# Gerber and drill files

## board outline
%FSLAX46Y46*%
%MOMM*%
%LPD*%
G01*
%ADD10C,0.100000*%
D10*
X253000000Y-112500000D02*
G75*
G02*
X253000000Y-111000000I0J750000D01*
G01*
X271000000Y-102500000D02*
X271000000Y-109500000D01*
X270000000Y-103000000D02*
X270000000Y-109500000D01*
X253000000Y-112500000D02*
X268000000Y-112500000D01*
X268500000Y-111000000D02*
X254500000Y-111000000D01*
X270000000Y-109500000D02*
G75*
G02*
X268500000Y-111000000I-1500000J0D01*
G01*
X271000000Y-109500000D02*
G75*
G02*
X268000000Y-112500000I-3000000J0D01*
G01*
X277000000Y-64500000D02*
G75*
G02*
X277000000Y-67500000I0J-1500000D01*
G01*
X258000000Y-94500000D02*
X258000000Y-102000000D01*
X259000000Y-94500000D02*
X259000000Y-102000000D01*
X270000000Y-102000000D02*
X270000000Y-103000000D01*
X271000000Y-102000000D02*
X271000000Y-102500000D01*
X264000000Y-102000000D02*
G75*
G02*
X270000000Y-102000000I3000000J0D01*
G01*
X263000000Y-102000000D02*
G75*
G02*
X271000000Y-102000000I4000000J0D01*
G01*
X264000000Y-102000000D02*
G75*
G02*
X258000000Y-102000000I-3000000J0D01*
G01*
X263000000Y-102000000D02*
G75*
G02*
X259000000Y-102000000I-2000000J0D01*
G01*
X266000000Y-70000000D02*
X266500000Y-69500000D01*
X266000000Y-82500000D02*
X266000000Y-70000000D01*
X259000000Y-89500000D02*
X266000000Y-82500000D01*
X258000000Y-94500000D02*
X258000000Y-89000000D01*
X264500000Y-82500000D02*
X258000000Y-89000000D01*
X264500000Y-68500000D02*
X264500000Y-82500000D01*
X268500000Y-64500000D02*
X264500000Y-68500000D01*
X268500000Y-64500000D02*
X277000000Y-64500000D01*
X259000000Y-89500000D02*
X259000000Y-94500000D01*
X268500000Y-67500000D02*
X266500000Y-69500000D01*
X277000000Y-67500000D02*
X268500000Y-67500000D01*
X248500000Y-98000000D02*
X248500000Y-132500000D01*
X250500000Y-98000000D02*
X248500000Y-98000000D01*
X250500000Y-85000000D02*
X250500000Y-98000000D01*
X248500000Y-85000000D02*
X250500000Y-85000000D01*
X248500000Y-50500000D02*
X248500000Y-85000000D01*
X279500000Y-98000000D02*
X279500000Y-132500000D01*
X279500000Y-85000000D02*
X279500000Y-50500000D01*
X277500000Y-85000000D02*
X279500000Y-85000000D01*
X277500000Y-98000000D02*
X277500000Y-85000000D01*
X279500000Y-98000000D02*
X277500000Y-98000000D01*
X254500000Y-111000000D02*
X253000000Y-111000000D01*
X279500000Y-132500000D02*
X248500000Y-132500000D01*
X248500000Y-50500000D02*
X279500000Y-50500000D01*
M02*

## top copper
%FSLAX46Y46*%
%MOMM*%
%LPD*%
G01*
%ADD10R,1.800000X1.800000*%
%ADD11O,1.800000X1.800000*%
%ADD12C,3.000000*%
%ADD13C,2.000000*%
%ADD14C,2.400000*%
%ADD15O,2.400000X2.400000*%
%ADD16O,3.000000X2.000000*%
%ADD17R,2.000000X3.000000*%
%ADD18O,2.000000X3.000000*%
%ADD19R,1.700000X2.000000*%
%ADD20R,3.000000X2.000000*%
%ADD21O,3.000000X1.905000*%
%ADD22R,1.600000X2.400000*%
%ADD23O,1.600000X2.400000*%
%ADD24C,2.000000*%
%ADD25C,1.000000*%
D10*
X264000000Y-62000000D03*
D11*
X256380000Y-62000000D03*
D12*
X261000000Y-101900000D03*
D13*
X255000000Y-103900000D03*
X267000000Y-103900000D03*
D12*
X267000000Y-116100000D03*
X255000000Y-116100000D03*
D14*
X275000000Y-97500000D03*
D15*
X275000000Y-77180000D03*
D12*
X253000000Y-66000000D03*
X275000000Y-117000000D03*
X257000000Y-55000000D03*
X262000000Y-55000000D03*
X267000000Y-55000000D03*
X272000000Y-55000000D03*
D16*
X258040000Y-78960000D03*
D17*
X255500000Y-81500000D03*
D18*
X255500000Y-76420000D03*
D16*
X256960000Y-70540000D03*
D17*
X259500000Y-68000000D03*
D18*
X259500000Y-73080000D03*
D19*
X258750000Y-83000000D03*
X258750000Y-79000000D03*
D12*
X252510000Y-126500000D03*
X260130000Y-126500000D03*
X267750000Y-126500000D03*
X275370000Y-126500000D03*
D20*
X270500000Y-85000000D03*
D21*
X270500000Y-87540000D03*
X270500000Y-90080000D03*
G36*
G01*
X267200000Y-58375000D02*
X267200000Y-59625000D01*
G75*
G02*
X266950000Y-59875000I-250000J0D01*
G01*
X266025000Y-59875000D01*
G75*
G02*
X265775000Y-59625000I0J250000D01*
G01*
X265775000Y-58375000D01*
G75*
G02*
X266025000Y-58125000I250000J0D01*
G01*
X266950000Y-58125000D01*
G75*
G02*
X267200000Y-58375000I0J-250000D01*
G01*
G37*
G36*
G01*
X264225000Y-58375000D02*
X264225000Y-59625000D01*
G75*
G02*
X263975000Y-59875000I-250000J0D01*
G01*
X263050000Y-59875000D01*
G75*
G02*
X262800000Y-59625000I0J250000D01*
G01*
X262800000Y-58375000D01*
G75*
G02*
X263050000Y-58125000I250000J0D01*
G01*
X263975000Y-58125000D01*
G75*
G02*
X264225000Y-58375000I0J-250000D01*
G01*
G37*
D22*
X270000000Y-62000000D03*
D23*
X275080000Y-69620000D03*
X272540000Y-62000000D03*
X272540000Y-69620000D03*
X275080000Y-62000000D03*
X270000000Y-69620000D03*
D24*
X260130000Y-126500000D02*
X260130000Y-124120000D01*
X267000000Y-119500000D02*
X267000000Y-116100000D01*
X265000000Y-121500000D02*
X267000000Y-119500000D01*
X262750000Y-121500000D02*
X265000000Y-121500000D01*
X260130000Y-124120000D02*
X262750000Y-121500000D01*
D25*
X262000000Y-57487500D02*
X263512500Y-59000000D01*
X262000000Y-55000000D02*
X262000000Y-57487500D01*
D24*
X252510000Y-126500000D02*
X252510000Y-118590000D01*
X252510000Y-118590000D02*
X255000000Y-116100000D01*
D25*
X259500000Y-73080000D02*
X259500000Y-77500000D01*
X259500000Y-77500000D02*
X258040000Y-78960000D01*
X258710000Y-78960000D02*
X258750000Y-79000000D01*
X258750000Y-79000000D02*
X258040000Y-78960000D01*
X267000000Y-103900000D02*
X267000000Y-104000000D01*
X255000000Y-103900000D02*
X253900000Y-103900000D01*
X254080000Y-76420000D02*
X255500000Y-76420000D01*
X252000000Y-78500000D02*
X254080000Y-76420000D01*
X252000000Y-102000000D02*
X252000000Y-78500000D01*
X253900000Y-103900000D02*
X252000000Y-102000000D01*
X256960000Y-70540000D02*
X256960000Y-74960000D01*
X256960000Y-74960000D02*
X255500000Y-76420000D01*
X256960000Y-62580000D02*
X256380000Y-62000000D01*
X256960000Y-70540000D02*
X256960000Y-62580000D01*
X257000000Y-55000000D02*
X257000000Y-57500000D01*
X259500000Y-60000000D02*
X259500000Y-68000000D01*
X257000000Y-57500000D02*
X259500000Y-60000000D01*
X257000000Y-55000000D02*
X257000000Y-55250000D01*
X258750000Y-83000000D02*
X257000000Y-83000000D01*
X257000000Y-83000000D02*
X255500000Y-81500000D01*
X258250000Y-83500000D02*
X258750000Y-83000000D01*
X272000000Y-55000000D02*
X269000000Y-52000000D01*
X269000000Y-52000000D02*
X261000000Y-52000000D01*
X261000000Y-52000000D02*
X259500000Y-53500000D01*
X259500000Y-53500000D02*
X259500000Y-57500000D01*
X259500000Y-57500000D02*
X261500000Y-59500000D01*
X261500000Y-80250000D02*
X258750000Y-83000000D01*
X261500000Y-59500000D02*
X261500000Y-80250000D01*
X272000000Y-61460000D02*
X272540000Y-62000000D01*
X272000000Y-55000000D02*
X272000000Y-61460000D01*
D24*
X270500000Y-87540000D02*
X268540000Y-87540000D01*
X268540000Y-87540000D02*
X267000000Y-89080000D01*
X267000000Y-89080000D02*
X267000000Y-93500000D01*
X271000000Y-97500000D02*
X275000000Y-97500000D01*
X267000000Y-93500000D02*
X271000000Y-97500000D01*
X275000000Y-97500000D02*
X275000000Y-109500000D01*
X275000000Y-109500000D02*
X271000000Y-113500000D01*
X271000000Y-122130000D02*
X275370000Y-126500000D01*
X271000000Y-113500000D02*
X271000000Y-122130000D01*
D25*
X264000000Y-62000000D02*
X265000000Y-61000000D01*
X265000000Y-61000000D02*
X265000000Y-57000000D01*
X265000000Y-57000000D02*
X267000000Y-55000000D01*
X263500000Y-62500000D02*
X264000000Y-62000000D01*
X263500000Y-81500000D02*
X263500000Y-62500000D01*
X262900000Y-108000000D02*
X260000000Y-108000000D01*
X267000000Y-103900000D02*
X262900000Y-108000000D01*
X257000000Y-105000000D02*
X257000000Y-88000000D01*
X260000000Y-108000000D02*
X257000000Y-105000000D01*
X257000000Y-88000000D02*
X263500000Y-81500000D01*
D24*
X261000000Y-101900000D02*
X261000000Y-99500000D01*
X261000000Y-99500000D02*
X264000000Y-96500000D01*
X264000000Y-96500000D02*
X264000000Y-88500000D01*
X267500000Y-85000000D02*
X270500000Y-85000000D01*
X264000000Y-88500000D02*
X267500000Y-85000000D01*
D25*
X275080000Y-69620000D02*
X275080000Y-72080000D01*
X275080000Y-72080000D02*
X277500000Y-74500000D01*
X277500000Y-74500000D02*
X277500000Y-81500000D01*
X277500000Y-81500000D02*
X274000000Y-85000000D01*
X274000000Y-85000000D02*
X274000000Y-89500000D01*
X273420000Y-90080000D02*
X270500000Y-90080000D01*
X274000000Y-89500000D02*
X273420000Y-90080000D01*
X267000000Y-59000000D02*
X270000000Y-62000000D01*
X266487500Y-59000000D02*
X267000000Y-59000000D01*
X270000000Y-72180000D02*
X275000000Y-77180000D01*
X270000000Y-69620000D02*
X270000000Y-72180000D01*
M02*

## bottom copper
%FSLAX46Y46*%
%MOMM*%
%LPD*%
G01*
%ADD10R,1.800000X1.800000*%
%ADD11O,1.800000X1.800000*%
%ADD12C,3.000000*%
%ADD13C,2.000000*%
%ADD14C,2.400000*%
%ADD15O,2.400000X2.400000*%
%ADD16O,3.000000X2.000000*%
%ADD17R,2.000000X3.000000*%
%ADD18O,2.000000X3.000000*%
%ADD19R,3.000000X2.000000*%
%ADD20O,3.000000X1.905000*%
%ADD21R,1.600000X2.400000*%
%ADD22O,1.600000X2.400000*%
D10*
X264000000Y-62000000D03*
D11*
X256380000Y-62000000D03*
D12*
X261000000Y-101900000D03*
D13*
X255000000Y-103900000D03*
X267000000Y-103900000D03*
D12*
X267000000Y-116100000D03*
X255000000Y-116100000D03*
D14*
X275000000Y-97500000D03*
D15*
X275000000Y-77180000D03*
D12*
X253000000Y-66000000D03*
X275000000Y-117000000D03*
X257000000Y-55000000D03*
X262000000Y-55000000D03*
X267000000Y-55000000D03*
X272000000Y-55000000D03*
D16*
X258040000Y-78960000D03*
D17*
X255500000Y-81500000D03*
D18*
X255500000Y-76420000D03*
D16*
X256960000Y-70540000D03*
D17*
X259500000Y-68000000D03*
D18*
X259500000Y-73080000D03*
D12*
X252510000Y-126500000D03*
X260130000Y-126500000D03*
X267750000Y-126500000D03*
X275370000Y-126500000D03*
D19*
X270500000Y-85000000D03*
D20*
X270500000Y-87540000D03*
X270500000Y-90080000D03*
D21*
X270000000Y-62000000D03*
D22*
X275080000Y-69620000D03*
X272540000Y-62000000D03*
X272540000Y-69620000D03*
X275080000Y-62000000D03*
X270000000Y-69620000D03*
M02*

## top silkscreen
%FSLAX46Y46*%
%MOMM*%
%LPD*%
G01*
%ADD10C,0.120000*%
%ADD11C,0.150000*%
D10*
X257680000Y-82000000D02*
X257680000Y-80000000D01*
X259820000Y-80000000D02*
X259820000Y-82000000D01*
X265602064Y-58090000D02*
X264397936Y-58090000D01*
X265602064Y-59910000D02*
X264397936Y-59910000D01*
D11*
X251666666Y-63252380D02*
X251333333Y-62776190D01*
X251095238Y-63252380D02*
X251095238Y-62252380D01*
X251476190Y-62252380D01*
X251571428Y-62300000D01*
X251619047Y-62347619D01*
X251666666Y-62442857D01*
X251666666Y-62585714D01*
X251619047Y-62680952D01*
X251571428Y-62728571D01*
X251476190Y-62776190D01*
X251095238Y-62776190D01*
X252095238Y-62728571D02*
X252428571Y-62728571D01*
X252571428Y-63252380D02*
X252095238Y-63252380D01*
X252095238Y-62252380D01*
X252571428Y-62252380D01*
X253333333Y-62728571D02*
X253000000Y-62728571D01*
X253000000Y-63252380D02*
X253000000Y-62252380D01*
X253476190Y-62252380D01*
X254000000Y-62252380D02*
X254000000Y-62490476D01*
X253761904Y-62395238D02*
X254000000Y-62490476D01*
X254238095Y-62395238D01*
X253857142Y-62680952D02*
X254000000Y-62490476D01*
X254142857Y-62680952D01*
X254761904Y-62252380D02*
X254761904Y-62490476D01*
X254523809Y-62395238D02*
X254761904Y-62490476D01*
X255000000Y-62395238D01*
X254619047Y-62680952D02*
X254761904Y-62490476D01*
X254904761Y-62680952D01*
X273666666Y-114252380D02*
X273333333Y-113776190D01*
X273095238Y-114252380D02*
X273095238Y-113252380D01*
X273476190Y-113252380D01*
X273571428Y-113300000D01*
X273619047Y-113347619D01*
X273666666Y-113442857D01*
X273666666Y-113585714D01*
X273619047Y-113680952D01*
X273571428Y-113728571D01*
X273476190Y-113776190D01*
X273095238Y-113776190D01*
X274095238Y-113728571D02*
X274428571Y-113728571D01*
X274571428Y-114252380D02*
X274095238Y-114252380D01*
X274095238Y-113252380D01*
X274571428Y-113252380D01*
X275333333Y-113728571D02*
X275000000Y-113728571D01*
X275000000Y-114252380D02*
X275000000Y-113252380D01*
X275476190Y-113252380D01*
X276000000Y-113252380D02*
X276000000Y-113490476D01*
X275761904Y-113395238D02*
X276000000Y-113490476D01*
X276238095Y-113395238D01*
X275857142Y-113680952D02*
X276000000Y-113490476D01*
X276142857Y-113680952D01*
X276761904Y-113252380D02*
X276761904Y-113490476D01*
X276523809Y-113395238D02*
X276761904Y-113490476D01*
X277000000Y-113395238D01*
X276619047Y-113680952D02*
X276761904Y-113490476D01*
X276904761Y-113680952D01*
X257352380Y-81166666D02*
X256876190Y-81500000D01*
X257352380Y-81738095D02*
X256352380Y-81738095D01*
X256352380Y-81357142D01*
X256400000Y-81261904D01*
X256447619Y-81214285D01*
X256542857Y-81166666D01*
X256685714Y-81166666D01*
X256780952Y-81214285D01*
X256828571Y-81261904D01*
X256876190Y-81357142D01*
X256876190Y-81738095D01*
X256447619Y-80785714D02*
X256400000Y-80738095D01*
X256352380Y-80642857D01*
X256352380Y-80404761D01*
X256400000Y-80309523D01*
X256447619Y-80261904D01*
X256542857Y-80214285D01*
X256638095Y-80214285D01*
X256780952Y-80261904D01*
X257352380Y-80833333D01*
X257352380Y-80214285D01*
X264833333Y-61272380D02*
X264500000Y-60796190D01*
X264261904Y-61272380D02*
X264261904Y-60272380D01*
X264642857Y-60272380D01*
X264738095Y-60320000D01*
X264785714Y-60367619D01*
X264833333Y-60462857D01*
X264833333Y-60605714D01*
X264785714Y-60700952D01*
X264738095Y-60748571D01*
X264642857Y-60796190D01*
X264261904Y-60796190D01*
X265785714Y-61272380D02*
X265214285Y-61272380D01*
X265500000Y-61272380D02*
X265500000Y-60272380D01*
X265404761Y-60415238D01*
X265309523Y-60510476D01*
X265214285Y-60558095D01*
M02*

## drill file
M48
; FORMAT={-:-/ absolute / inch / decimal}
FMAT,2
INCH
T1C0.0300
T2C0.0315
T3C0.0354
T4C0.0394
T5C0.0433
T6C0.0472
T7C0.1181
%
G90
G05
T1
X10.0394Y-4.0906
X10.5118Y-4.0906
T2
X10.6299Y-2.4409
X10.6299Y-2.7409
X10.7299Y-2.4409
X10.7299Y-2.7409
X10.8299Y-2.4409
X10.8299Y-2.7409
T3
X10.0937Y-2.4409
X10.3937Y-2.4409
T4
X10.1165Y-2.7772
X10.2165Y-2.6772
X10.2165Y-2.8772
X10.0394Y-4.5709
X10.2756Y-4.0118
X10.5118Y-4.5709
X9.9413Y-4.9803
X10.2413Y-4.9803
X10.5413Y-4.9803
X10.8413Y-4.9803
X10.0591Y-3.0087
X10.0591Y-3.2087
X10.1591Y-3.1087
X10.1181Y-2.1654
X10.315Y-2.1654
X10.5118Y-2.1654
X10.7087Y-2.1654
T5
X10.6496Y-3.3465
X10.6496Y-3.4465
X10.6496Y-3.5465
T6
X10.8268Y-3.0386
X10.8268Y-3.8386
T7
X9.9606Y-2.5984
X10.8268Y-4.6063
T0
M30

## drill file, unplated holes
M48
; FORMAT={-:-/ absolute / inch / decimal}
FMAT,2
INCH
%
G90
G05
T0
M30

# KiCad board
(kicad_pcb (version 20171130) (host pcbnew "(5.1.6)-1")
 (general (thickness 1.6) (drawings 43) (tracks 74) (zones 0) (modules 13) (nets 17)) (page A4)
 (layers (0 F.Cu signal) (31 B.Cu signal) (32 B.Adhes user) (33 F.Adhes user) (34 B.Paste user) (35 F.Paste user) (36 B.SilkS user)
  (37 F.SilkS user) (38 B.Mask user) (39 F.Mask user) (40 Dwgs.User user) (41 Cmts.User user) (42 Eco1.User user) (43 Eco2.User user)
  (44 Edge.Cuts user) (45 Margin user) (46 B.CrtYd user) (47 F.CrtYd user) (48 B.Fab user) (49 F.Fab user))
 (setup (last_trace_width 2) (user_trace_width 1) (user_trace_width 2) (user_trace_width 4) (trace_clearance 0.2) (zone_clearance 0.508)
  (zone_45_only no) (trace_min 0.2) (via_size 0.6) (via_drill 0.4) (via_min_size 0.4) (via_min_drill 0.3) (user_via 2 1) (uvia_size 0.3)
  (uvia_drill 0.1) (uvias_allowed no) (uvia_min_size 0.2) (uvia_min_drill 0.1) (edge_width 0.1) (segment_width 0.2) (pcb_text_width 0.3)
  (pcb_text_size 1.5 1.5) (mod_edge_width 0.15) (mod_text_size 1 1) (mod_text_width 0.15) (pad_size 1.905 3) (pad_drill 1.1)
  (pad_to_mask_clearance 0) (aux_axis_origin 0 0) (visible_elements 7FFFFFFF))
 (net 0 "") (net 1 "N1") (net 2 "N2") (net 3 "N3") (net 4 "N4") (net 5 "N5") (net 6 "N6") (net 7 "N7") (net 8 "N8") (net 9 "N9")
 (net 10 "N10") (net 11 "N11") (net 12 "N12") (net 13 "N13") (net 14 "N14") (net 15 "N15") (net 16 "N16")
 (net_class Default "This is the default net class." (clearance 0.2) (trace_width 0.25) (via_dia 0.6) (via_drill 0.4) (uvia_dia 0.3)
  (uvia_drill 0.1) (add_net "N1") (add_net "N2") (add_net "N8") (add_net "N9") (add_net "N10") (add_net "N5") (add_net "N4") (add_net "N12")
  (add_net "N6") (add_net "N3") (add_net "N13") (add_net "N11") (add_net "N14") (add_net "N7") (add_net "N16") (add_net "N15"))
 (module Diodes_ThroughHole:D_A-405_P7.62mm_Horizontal (layer B.Cu) (at 264 62 180)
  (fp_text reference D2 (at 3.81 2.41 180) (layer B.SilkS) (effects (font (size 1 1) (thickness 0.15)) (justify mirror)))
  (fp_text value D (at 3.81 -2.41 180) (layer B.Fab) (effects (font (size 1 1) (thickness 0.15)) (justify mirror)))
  (pad 1 thru_hole rect (at 0 0 180) (size 1.8 1.8) (drill 0.9) (layers *.Cu *.Mask) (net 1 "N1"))
  (pad 2 thru_hole oval (at 7.62 0 180) (size 1.8 1.8) (drill 0.9) (layers *.Cu *.Mask) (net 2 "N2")))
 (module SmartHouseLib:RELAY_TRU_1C (layer B.Cu) (at 261 110 270)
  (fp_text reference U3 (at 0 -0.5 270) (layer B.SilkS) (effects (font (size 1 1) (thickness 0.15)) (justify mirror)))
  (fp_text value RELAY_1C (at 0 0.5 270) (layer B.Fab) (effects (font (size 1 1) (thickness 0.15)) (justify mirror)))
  (pad 3 thru_hole circle (at -8.1 0 270) (size 3 3) (drill 1) (layers *.Cu *.Mask) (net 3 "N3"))
  (pad 1 thru_hole circle (at -6.1 6 270) (size 2 2) (drill 0.762) (layers *.Cu *.Mask) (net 2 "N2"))
  (pad 2 thru_hole circle (at -6.1 -6 270) (size 2 2) (drill 0.762) (layers *.Cu *.Mask) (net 1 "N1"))
  (pad 5 thru_hole circle (at 6.1 -6 270) (size 3 3) (drill 1) (layers *.Cu *.Mask) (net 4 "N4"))
  (pad 4 thru_hole circle (at 6.1 6 270) (size 3 3) (drill 1) (layers *.Cu *.Mask) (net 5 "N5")))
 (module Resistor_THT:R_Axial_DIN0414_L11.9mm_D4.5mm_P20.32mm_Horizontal (layer B.Cu) (at 275 97.5 90)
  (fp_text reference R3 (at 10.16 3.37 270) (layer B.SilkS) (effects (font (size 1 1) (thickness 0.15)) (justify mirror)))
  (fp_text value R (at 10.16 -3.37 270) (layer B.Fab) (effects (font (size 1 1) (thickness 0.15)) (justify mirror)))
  (pad 1 thru_hole circle (at 0 0 90) (size 2.4 2.4) (drill 1.2) (layers *.Cu *.Mask) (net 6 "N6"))
  (pad 2 thru_hole oval (at 20.32 0 90) (size 2.4 2.4) (drill 1.2) (layers *.Cu *.Mask) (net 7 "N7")))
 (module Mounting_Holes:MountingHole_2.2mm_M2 (layer F.Cu) (at 253 66)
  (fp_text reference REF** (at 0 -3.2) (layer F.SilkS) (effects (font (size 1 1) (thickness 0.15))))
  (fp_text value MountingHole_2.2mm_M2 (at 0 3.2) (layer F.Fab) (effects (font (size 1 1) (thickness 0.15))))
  (pad 1 thru_hole circle (at 0 0) (size 3 3) (drill 3) (layers *.Cu *.Mask)))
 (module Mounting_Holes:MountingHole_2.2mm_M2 (layer F.Cu) (at 275 117)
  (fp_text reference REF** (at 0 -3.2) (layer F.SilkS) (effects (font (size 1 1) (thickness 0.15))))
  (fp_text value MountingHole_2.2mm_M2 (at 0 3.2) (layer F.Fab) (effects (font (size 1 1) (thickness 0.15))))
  (pad 1 thru_hole circle (at 0 0) (size 3 3) (drill 3) (layers *.Cu *.Mask)))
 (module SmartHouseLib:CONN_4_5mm (layer B.Cu) (at 267 55)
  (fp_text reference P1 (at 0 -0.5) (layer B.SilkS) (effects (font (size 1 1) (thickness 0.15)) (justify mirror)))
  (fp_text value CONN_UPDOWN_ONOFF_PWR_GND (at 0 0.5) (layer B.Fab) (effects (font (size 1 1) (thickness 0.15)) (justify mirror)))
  (pad 1 thru_hole circle (at -10 0) (size 3 3) (drill 1) (layers *.Cu *.Mask) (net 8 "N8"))
  (pad 2 thru_hole circle (at -5 0) (size 3 3) (drill 1) (layers *.Cu *.Mask) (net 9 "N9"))
  (pad 3 thru_hole circle (at 0 0) (size 3 3) (drill 1) (layers *.Cu *.Mask) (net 1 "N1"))
  (pad 4 thru_hole circle (at 5 0) (size 3 3) (drill 1) (layers *.Cu *.Mask) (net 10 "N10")))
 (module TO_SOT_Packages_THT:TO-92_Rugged (layer B.Cu) (at 255.5 81.5 90)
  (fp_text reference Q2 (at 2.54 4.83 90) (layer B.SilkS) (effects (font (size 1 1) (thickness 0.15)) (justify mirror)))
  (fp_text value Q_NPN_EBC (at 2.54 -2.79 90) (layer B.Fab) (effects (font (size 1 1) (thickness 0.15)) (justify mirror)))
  (pad 2 thru_hole oval (at 2.54 2.54) (size 3 2) (drill 1) (layers *.Cu *.Mask) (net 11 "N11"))
  (pad 1 thru_hole rect (at 0 0) (size 2 3) (drill 1) (layers *.Cu *.Mask) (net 10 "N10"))
  (pad 3 thru_hole oval (at 5.08 0) (size 2 3) (drill 1) (layers *.Cu *.Mask) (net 2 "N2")))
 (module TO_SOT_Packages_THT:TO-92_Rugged (layer B.Cu) (at 259.5 68 270)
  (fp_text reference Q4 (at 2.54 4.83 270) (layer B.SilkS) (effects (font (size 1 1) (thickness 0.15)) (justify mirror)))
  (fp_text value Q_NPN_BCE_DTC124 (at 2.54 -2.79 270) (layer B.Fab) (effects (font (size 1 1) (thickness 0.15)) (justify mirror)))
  (pad 2 thru_hole oval (at 2.54 2.54 180) (size 3 2) (drill 1) (layers *.Cu *.Mask) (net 2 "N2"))
  (pad 1 thru_hole rect (at 0 0 180) (size 2 3) (drill 1) (layers *.Cu *.Mask) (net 8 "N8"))
  (pad 3 thru_hole oval (at 5.08 0 180) (size 2 3) (drill 1) (layers *.Cu *.Mask) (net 11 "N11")))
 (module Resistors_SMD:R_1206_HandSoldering (layer F.Cu) (at 258.75 81 90)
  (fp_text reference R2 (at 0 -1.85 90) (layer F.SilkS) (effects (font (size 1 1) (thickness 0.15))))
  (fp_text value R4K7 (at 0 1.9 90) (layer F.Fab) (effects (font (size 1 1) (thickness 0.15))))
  (fp_line (start -1 -1.07) (end 1 -1.07) (layer F.SilkS) (width 0.12))
  (fp_line (start 1 1.07) (end -1 1.07) (layer F.SilkS) (width 0.12))
  (pad 1 smd rect (at -2 0 90) (size 2 1.7) (layers F.Cu F.Paste F.Mask) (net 10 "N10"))
  (pad 2 smd rect (at 2 0 90) (size 2 1.7) (layers F.Cu F.Paste F.Mask) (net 11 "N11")))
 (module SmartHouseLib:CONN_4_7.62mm (layer B.Cu) (at 267.75 126.5)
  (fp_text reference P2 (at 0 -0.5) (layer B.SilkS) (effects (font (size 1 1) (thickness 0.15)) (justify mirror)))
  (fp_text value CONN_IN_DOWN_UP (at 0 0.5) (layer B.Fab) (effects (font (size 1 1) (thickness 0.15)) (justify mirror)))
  (pad 1 thru_hole circle (at -15.24 0) (size 3 3) (drill 1) (layers *.Cu *.Mask) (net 5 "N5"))
  (pad 2 thru_hole circle (at -7.62 0) (size 3 3) (drill 1) (layers *.Cu *.Mask) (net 4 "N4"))
  (pad 3 thru_hole circle (at 0 0) (size 3 3) (drill 1) (layers *.Cu *.Mask) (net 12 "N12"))
  (pad 4 thru_hole circle (at 7.62 0) (size 3 3) (drill 1) (layers *.Cu *.Mask) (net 6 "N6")))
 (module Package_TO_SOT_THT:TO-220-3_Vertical (layer B.Cu) (at 270.5 85 270)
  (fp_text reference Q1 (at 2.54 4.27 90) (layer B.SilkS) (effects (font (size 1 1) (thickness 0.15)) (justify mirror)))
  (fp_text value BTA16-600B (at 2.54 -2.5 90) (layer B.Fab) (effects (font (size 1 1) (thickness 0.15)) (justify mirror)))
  (pad 1 thru_hole rect (at 0 0 270) (size 2 3) (drill 1.1) (layers *.Cu *.Mask) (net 3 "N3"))
  (pad 2 thru_hole oval (at 2.54 0 270) (size 1.905 3) (drill 1.1) (layers *.Cu *.Mask) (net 6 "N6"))
  (pad 3 thru_hole oval (at 5.08 0 270) (size 1.905 3) (drill 1.1) (layers *.Cu *.Mask) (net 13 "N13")))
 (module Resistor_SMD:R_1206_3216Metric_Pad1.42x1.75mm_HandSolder (layer F.Cu) (at 265 59 180)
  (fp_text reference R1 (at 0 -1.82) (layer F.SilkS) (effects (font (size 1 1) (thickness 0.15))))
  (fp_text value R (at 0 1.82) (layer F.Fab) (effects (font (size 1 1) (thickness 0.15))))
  (fp_line (start -0.602064 0.91) (end 0.602064 0.91) (layer F.SilkS) (width 0.12))
  (fp_line (start -0.602064 -0.91) (end 0.602064 -0.91) (layer F.SilkS) (width 0.12))
  (pad 1 smd roundrect (at -1.4875 0 180) (size 1.425 1.75) (layers F.Cu F.Paste F.Mask) (roundrect_rratio 0.175439) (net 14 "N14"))
  (pad 2 smd roundrect (at 1.4875 0 180) (size 1.425 1.75) (layers F.Cu F.Paste F.Mask) (roundrect_rratio 0.175439) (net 9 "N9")))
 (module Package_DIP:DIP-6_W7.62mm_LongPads (layer B.Cu) (at 270 62 270)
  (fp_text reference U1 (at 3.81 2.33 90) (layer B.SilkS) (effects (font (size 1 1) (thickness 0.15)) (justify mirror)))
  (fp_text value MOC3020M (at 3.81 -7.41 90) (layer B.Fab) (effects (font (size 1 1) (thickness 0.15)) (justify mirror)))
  (pad 1 thru_hole rect (at 0 0 270) (size 2.4 1.6) (drill 0.8) (layers *.Cu *.Mask) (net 14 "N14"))
  (pad 4 thru_hole oval (at 7.62 -5.08 270) (size 2.4 1.6) (drill 0.8) (layers *.Cu *.Mask) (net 13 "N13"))
  (pad 2 thru_hole oval (at 0 -2.54 270) (size 2.4 1.6) (drill 0.8) (layers *.Cu *.Mask) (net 10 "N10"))
  (pad 5 thru_hole oval (at 7.62 -2.54 270) (size 2.4 1.6) (drill 0.8) (layers *.Cu *.Mask) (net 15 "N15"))
  (pad 3 thru_hole oval (at 0 -5.08 270) (size 2.4 1.6) (drill 0.8) (layers *.Cu *.Mask) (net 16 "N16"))
  (pad 6 thru_hole oval (at 7.62 0 270) (size 2.4 1.6) (drill 0.8) (layers *.Cu *.Mask) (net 7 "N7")))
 (gr_arc (start 253 111.75) (end 253 111) (angle -180) (layer Edge.Cuts) (width 0.1))
 (gr_line (start 271 102.5) (end 271 109.5) (layer Edge.Cuts) (width 0.1))
 (gr_line (start 270 103) (end 270 109.5) (layer Edge.Cuts) (width 0.1))
 (gr_line (start 253 112.5) (end 268 112.5) (layer Edge.Cuts) (width 0.1))
 (gr_line (start 268.5 111) (end 254.5 111) (layer Edge.Cuts) (width 0.1))
 (gr_arc (start 268.5 109.5) (end 268.5 111) (angle -90) (layer Edge.Cuts) (width 0.1))
 (gr_arc (start 268 109.5) (end 268 112.5) (angle -90) (layer Edge.Cuts) (width 0.1))
 (gr_arc (start 277 66) (end 277 67.5) (angle -180) (layer Edge.Cuts) (width 0.1))
 (gr_line (start 258 94.5) (end 258 102) (layer Edge.Cuts) (width 0.1))
 (gr_line (start 259 94.5) (end 259 102) (layer Edge.Cuts) (width 0.1))
 (gr_line (start 270 102) (end 270 103) (layer Edge.Cuts) (width 0.1))
 (gr_line (start 271 102) (end 271 102.5) (layer Edge.Cuts) (width 0.1))
 (gr_arc (start 267 102) (end 270 102) (angle -180) (layer Edge.Cuts) (width 0.1))
 (gr_arc (start 267 102) (end 271 102) (angle -180) (layer Edge.Cuts) (width 0.1))
 (gr_arc (start 261 102) (end 258 102) (angle -180) (layer Edge.Cuts) (width 0.1))
 (gr_arc (start 261 102) (end 259 102) (angle -180) (layer Edge.Cuts) (width 0.1))
 (gr_line (start 266 70) (end 266.5 69.5) (layer Edge.Cuts) (width 0.1))
 (gr_line (start 266 82.5) (end 266 70) (layer Edge.Cuts) (width 0.1))
 (gr_line (start 259 89.5) (end 266 82.5) (layer Edge.Cuts) (width 0.1))
 (gr_line (start 258 94.5) (end 258 89) (layer Edge.Cuts) (width 0.1))
 (gr_line (start 264.5 82.5) (end 258 89) (layer Edge.Cuts) (width 0.1))
 (gr_line (start 264.5 68.5) (end 264.5 82.5) (layer Edge.Cuts) (width 0.1))
 (gr_line (start 268.5 64.5) (end 264.5 68.5) (layer Edge.Cuts) (width 0.1))
 (gr_line (start 268.5 64.5) (end 277 64.5) (layer Edge.Cuts) (width 0.1))
 (gr_line (start 259 89.5) (end 259 94.5) (layer Edge.Cuts) (width 0.1))
 (gr_line (start 268.5 67.5) (end 266.5 69.5) (layer Edge.Cuts) (width 0.1))
 (gr_line (start 277 67.5) (end 268.5 67.5) (layer Edge.Cuts) (width 0.1))
 (gr_line (start 248.5 98) (end 248.5 132.5) (angle 90) (layer Edge.Cuts) (width 0.1))
 (gr_line (start 250.5 98) (end 248.5 98) (angle 90) (layer Edge.Cuts) (width 0.1))
 (gr_line (start 250.5 85) (end 250.5 98) (angle 90) (layer Edge.Cuts) (width 0.1))
 (gr_line (start 248.5 85) (end 250.5 85) (angle 90) (layer Edge.Cuts) (width 0.1))
 (gr_line (start 248.5 50.5) (end 248.5 85) (angle 90) (layer Edge.Cuts) (width 0.1))
 (gr_line (start 279.5 98) (end 279.5 132.5) (angle 90) (layer Edge.Cuts) (width 0.1))
 (gr_line (start 279.5 85) (end 279.5 50.5) (angle 90) (layer Edge.Cuts) (width 0.1))
 (gr_line (start 277.5 85) (end 279.5 85) (angle 90) (layer Edge.Cuts) (width 0.1))
 (gr_line (start 277.5 98) (end 277.5 85) (angle 90) (layer Edge.Cuts) (width 0.1))
 (gr_line (start 279.5 98) (end 277.5 98) (angle 90) (layer Edge.Cuts) (width 0.1))
 (gr_line (start 254.5 111) (end 253 111) (angle 90) (layer Edge.Cuts) (width 0.1))
 (gr_line (start 279.5 132.5) (end 248.5 132.5) (angle 90) (layer Edge.Cuts) (width 0.1))
 (gr_line (start 248.5 50.5) (end 279.5 50.5) (angle 90) (layer Edge.Cuts) (width 0.1))
 (segment (start 260.13 126.5) (end 260.13 124.12) (width 2) (layer F.Cu) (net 4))
 (segment (start 267 119.5) (end 267 116.1) (width 2) (layer F.Cu) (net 4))
 (segment (start 265 121.5) (end 267 119.5) (width 2) (layer F.Cu) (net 4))
 (segment (start 262.75 121.5) (end 265 121.5) (width 2) (layer F.Cu) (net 4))
 (segment (start 260.13 124.12) (end 262.75 121.5) (width 2) (layer F.Cu) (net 4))
 (segment (start 262 57.4875) (end 263.5125 59) (width 1) (layer F.Cu) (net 9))
 (segment (start 262 55) (end 262 57.4875) (width 1) (layer F.Cu) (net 9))
 (segment (start 252.51 126.5) (end 252.51 118.59) (width 2) (layer F.Cu) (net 5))
 (segment (start 252.51 118.59) (end 255 116.1) (width 2) (layer F.Cu) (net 5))
 (segment (start 259.5 73.08) (end 259.5 77.5) (width 1) (layer F.Cu) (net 11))
 (segment (start 259.5 77.5) (end 258.04 78.96) (width 1) (layer F.Cu) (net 11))
 (segment (start 258.71 78.96) (end 258.75 79) (width 1) (layer F.Cu) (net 11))
 (segment (start 258.75 79) (end 258.04 78.96) (width 1) (layer F.Cu) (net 11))
 (segment (start 267 103.9) (end 267 104) (width 1) (layer F.Cu) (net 1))
 (segment (start 255 103.9) (end 253.9 103.9) (width 1) (layer F.Cu) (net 2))
 (segment (start 254.08 76.42) (end 255.5 76.42) (width 1) (layer F.Cu) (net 2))
 (segment (start 252 78.5) (end 254.08 76.42) (width 1) (layer F.Cu) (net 2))
 (segment (start 252 102) (end 252 78.5) (width 1) (layer F.Cu) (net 2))
 (segment (start 253.9 103.9) (end 252 102) (width 1) (layer F.Cu) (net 2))
 (segment (start 256.96 70.54) (end 256.96 74.96) (width 1) (layer F.Cu) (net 2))
 (segment (start 256.96 74.96) (end 255.5 76.42) (width 1) (layer F.Cu) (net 2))
 (segment (start 256.96 62.58) (end 256.38 62) (width 1) (layer F.Cu) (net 2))
 (segment (start 256.96 70.54) (end 256.96 62.58) (width 1) (layer F.Cu) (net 2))
 (segment (start 257 55) (end 257 57.5) (width 1) (layer F.Cu) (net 8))
 (segment (start 259.5 60) (end 259.5 68) (width 1) (layer F.Cu) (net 8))
 (segment (start 257 57.5) (end 259.5 60) (width 1) (layer F.Cu) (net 8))
 (segment (start 257 55) (end 257 55.25) (width 1) (layer F.Cu) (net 8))
 (segment (start 258.75 83) (end 257 83) (width 1) (layer F.Cu) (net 10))
 (segment (start 257 83) (end 255.5 81.5) (width 1) (layer F.Cu) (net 10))
 (segment (start 258.25 83.5) (end 258.75 83) (width 1) (layer F.Cu) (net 10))
 (segment (start 272 55) (end 269 52) (width 1) (layer F.Cu) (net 10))
 (segment (start 269 52) (end 261 52) (width 1) (layer F.Cu) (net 10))
 (segment (start 261 52) (end 259.5 53.5) (width 1) (layer F.Cu) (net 10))
 (segment (start 259.5 53.5) (end 259.5 57.5) (width 1) (layer F.Cu) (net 10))
 (segment (start 259.5 57.5) (end 261.5 59.5) (width 1) (layer F.Cu) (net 10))
 (segment (start 261.5 80.25) (end 258.75 83) (width 1) (layer F.Cu) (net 10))
 (segment (start 261.5 59.5) (end 261.5 80.25) (width 1) (layer F.Cu) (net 10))
 (segment (start 272 61.46) (end 272.54 62) (width 1) (layer F.Cu) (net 10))
 (segment (start 272 55) (end 272 61.46) (width 1) (layer F.Cu) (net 10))
 (segment (start 270.5 87.54) (end 268.54 87.54) (width 2) (layer F.Cu) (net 6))
 (segment (start 268.54 87.54) (end 267 89.08) (width 2) (layer F.Cu) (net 6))
 (segment (start 267 89.08) (end 267 93.5) (width 2) (layer F.Cu) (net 6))
 (segment (start 271 97.5) (end 275 97.5) (width 2) (layer F.Cu) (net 6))
 (segment (start 267 93.5) (end 271 97.5) (width 2) (layer F.Cu) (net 6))
 (segment (start 275 97.5) (end 275 109.5) (width 2) (layer F.Cu) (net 6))
 (segment (start 275 109.5) (end 271 113.5) (width 2) (layer F.Cu) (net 6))
 (segment (start 271 122.13) (end 275.37 126.5) (width 2) (layer F.Cu) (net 6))
 (segment (start 271 113.5) (end 271 122.13) (width 2) (layer F.Cu) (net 6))
 (segment (start 264 62) (end 265 61) (width 1) (layer F.Cu) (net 1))
 (segment (start 265 61) (end 265 57) (width 1) (layer F.Cu) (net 1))
 (segment (start 265 57) (end 267 55) (width 1) (layer F.Cu) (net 1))
 (segment (start 263.5 62.5) (end 264 62) (width 1) (layer F.Cu) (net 1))
 (segment (start 263.5 81.5) (end 263.5 62.5) (width 1) (layer F.Cu) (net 1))
 (segment (start 262.9 108) (end 260 108) (width 1) (layer F.Cu) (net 1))
 (segment (start 267 103.9) (end 262.9 108) (width 1) (layer F.Cu) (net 1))
 (segment (start 257 105) (end 257 88) (width 1) (layer F.Cu) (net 1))
 (segment (start 260 108) (end 257 105) (width 1) (layer F.Cu) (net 1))
 (segment (start 257 88) (end 263.5 81.5) (width 1) (layer F.Cu) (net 1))
 (segment (start 261 101.9) (end 261 99.5) (width 2) (layer F.Cu) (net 3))
 (segment (start 261 99.5) (end 264 96.5) (width 2) (layer F.Cu) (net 3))
 (segment (start 264 96.5) (end 264 88.5) (width 2) (layer F.Cu) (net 3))
 (segment (start 267.5 85) (end 270.5 85) (width 2) (layer F.Cu) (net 3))
 (segment (start 264 88.5) (end 267.5 85) (width 2) (layer F.Cu) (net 3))
 (segment (start 275.08 69.62) (end 275.08 72.08) (width 1) (layer F.Cu) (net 13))
 (segment (start 275.08 72.08) (end 277.5 74.5) (width 1) (layer F.Cu) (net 13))
 (segment (start 277.5 74.5) (end 277.5 81.5) (width 1) (layer F.Cu) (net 13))
 (segment (start 277.5 81.5) (end 274 85) (width 1) (layer F.Cu) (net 13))
 (segment (start 274 85) (end 274 89.5) (width 1) (layer F.Cu) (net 13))
 (segment (start 273.42 90.08) (end 270.5 90.08) (width 1) (layer F.Cu) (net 13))
 (segment (start 274 89.5) (end 273.42 90.08) (width 1) (layer F.Cu) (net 13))
 (segment (start 267 59) (end 270 62) (width 1) (layer F.Cu) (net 14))
 (segment (start 266.4875 59) (end 267 59) (width 1) (layer F.Cu) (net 14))
 (segment (start 270 72.18) (end 275 77.18) (width 1) (layer F.Cu) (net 7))
 (segment (start 270 69.62) (end 270 72.18) (width 1) (layer F.Cu) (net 7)))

